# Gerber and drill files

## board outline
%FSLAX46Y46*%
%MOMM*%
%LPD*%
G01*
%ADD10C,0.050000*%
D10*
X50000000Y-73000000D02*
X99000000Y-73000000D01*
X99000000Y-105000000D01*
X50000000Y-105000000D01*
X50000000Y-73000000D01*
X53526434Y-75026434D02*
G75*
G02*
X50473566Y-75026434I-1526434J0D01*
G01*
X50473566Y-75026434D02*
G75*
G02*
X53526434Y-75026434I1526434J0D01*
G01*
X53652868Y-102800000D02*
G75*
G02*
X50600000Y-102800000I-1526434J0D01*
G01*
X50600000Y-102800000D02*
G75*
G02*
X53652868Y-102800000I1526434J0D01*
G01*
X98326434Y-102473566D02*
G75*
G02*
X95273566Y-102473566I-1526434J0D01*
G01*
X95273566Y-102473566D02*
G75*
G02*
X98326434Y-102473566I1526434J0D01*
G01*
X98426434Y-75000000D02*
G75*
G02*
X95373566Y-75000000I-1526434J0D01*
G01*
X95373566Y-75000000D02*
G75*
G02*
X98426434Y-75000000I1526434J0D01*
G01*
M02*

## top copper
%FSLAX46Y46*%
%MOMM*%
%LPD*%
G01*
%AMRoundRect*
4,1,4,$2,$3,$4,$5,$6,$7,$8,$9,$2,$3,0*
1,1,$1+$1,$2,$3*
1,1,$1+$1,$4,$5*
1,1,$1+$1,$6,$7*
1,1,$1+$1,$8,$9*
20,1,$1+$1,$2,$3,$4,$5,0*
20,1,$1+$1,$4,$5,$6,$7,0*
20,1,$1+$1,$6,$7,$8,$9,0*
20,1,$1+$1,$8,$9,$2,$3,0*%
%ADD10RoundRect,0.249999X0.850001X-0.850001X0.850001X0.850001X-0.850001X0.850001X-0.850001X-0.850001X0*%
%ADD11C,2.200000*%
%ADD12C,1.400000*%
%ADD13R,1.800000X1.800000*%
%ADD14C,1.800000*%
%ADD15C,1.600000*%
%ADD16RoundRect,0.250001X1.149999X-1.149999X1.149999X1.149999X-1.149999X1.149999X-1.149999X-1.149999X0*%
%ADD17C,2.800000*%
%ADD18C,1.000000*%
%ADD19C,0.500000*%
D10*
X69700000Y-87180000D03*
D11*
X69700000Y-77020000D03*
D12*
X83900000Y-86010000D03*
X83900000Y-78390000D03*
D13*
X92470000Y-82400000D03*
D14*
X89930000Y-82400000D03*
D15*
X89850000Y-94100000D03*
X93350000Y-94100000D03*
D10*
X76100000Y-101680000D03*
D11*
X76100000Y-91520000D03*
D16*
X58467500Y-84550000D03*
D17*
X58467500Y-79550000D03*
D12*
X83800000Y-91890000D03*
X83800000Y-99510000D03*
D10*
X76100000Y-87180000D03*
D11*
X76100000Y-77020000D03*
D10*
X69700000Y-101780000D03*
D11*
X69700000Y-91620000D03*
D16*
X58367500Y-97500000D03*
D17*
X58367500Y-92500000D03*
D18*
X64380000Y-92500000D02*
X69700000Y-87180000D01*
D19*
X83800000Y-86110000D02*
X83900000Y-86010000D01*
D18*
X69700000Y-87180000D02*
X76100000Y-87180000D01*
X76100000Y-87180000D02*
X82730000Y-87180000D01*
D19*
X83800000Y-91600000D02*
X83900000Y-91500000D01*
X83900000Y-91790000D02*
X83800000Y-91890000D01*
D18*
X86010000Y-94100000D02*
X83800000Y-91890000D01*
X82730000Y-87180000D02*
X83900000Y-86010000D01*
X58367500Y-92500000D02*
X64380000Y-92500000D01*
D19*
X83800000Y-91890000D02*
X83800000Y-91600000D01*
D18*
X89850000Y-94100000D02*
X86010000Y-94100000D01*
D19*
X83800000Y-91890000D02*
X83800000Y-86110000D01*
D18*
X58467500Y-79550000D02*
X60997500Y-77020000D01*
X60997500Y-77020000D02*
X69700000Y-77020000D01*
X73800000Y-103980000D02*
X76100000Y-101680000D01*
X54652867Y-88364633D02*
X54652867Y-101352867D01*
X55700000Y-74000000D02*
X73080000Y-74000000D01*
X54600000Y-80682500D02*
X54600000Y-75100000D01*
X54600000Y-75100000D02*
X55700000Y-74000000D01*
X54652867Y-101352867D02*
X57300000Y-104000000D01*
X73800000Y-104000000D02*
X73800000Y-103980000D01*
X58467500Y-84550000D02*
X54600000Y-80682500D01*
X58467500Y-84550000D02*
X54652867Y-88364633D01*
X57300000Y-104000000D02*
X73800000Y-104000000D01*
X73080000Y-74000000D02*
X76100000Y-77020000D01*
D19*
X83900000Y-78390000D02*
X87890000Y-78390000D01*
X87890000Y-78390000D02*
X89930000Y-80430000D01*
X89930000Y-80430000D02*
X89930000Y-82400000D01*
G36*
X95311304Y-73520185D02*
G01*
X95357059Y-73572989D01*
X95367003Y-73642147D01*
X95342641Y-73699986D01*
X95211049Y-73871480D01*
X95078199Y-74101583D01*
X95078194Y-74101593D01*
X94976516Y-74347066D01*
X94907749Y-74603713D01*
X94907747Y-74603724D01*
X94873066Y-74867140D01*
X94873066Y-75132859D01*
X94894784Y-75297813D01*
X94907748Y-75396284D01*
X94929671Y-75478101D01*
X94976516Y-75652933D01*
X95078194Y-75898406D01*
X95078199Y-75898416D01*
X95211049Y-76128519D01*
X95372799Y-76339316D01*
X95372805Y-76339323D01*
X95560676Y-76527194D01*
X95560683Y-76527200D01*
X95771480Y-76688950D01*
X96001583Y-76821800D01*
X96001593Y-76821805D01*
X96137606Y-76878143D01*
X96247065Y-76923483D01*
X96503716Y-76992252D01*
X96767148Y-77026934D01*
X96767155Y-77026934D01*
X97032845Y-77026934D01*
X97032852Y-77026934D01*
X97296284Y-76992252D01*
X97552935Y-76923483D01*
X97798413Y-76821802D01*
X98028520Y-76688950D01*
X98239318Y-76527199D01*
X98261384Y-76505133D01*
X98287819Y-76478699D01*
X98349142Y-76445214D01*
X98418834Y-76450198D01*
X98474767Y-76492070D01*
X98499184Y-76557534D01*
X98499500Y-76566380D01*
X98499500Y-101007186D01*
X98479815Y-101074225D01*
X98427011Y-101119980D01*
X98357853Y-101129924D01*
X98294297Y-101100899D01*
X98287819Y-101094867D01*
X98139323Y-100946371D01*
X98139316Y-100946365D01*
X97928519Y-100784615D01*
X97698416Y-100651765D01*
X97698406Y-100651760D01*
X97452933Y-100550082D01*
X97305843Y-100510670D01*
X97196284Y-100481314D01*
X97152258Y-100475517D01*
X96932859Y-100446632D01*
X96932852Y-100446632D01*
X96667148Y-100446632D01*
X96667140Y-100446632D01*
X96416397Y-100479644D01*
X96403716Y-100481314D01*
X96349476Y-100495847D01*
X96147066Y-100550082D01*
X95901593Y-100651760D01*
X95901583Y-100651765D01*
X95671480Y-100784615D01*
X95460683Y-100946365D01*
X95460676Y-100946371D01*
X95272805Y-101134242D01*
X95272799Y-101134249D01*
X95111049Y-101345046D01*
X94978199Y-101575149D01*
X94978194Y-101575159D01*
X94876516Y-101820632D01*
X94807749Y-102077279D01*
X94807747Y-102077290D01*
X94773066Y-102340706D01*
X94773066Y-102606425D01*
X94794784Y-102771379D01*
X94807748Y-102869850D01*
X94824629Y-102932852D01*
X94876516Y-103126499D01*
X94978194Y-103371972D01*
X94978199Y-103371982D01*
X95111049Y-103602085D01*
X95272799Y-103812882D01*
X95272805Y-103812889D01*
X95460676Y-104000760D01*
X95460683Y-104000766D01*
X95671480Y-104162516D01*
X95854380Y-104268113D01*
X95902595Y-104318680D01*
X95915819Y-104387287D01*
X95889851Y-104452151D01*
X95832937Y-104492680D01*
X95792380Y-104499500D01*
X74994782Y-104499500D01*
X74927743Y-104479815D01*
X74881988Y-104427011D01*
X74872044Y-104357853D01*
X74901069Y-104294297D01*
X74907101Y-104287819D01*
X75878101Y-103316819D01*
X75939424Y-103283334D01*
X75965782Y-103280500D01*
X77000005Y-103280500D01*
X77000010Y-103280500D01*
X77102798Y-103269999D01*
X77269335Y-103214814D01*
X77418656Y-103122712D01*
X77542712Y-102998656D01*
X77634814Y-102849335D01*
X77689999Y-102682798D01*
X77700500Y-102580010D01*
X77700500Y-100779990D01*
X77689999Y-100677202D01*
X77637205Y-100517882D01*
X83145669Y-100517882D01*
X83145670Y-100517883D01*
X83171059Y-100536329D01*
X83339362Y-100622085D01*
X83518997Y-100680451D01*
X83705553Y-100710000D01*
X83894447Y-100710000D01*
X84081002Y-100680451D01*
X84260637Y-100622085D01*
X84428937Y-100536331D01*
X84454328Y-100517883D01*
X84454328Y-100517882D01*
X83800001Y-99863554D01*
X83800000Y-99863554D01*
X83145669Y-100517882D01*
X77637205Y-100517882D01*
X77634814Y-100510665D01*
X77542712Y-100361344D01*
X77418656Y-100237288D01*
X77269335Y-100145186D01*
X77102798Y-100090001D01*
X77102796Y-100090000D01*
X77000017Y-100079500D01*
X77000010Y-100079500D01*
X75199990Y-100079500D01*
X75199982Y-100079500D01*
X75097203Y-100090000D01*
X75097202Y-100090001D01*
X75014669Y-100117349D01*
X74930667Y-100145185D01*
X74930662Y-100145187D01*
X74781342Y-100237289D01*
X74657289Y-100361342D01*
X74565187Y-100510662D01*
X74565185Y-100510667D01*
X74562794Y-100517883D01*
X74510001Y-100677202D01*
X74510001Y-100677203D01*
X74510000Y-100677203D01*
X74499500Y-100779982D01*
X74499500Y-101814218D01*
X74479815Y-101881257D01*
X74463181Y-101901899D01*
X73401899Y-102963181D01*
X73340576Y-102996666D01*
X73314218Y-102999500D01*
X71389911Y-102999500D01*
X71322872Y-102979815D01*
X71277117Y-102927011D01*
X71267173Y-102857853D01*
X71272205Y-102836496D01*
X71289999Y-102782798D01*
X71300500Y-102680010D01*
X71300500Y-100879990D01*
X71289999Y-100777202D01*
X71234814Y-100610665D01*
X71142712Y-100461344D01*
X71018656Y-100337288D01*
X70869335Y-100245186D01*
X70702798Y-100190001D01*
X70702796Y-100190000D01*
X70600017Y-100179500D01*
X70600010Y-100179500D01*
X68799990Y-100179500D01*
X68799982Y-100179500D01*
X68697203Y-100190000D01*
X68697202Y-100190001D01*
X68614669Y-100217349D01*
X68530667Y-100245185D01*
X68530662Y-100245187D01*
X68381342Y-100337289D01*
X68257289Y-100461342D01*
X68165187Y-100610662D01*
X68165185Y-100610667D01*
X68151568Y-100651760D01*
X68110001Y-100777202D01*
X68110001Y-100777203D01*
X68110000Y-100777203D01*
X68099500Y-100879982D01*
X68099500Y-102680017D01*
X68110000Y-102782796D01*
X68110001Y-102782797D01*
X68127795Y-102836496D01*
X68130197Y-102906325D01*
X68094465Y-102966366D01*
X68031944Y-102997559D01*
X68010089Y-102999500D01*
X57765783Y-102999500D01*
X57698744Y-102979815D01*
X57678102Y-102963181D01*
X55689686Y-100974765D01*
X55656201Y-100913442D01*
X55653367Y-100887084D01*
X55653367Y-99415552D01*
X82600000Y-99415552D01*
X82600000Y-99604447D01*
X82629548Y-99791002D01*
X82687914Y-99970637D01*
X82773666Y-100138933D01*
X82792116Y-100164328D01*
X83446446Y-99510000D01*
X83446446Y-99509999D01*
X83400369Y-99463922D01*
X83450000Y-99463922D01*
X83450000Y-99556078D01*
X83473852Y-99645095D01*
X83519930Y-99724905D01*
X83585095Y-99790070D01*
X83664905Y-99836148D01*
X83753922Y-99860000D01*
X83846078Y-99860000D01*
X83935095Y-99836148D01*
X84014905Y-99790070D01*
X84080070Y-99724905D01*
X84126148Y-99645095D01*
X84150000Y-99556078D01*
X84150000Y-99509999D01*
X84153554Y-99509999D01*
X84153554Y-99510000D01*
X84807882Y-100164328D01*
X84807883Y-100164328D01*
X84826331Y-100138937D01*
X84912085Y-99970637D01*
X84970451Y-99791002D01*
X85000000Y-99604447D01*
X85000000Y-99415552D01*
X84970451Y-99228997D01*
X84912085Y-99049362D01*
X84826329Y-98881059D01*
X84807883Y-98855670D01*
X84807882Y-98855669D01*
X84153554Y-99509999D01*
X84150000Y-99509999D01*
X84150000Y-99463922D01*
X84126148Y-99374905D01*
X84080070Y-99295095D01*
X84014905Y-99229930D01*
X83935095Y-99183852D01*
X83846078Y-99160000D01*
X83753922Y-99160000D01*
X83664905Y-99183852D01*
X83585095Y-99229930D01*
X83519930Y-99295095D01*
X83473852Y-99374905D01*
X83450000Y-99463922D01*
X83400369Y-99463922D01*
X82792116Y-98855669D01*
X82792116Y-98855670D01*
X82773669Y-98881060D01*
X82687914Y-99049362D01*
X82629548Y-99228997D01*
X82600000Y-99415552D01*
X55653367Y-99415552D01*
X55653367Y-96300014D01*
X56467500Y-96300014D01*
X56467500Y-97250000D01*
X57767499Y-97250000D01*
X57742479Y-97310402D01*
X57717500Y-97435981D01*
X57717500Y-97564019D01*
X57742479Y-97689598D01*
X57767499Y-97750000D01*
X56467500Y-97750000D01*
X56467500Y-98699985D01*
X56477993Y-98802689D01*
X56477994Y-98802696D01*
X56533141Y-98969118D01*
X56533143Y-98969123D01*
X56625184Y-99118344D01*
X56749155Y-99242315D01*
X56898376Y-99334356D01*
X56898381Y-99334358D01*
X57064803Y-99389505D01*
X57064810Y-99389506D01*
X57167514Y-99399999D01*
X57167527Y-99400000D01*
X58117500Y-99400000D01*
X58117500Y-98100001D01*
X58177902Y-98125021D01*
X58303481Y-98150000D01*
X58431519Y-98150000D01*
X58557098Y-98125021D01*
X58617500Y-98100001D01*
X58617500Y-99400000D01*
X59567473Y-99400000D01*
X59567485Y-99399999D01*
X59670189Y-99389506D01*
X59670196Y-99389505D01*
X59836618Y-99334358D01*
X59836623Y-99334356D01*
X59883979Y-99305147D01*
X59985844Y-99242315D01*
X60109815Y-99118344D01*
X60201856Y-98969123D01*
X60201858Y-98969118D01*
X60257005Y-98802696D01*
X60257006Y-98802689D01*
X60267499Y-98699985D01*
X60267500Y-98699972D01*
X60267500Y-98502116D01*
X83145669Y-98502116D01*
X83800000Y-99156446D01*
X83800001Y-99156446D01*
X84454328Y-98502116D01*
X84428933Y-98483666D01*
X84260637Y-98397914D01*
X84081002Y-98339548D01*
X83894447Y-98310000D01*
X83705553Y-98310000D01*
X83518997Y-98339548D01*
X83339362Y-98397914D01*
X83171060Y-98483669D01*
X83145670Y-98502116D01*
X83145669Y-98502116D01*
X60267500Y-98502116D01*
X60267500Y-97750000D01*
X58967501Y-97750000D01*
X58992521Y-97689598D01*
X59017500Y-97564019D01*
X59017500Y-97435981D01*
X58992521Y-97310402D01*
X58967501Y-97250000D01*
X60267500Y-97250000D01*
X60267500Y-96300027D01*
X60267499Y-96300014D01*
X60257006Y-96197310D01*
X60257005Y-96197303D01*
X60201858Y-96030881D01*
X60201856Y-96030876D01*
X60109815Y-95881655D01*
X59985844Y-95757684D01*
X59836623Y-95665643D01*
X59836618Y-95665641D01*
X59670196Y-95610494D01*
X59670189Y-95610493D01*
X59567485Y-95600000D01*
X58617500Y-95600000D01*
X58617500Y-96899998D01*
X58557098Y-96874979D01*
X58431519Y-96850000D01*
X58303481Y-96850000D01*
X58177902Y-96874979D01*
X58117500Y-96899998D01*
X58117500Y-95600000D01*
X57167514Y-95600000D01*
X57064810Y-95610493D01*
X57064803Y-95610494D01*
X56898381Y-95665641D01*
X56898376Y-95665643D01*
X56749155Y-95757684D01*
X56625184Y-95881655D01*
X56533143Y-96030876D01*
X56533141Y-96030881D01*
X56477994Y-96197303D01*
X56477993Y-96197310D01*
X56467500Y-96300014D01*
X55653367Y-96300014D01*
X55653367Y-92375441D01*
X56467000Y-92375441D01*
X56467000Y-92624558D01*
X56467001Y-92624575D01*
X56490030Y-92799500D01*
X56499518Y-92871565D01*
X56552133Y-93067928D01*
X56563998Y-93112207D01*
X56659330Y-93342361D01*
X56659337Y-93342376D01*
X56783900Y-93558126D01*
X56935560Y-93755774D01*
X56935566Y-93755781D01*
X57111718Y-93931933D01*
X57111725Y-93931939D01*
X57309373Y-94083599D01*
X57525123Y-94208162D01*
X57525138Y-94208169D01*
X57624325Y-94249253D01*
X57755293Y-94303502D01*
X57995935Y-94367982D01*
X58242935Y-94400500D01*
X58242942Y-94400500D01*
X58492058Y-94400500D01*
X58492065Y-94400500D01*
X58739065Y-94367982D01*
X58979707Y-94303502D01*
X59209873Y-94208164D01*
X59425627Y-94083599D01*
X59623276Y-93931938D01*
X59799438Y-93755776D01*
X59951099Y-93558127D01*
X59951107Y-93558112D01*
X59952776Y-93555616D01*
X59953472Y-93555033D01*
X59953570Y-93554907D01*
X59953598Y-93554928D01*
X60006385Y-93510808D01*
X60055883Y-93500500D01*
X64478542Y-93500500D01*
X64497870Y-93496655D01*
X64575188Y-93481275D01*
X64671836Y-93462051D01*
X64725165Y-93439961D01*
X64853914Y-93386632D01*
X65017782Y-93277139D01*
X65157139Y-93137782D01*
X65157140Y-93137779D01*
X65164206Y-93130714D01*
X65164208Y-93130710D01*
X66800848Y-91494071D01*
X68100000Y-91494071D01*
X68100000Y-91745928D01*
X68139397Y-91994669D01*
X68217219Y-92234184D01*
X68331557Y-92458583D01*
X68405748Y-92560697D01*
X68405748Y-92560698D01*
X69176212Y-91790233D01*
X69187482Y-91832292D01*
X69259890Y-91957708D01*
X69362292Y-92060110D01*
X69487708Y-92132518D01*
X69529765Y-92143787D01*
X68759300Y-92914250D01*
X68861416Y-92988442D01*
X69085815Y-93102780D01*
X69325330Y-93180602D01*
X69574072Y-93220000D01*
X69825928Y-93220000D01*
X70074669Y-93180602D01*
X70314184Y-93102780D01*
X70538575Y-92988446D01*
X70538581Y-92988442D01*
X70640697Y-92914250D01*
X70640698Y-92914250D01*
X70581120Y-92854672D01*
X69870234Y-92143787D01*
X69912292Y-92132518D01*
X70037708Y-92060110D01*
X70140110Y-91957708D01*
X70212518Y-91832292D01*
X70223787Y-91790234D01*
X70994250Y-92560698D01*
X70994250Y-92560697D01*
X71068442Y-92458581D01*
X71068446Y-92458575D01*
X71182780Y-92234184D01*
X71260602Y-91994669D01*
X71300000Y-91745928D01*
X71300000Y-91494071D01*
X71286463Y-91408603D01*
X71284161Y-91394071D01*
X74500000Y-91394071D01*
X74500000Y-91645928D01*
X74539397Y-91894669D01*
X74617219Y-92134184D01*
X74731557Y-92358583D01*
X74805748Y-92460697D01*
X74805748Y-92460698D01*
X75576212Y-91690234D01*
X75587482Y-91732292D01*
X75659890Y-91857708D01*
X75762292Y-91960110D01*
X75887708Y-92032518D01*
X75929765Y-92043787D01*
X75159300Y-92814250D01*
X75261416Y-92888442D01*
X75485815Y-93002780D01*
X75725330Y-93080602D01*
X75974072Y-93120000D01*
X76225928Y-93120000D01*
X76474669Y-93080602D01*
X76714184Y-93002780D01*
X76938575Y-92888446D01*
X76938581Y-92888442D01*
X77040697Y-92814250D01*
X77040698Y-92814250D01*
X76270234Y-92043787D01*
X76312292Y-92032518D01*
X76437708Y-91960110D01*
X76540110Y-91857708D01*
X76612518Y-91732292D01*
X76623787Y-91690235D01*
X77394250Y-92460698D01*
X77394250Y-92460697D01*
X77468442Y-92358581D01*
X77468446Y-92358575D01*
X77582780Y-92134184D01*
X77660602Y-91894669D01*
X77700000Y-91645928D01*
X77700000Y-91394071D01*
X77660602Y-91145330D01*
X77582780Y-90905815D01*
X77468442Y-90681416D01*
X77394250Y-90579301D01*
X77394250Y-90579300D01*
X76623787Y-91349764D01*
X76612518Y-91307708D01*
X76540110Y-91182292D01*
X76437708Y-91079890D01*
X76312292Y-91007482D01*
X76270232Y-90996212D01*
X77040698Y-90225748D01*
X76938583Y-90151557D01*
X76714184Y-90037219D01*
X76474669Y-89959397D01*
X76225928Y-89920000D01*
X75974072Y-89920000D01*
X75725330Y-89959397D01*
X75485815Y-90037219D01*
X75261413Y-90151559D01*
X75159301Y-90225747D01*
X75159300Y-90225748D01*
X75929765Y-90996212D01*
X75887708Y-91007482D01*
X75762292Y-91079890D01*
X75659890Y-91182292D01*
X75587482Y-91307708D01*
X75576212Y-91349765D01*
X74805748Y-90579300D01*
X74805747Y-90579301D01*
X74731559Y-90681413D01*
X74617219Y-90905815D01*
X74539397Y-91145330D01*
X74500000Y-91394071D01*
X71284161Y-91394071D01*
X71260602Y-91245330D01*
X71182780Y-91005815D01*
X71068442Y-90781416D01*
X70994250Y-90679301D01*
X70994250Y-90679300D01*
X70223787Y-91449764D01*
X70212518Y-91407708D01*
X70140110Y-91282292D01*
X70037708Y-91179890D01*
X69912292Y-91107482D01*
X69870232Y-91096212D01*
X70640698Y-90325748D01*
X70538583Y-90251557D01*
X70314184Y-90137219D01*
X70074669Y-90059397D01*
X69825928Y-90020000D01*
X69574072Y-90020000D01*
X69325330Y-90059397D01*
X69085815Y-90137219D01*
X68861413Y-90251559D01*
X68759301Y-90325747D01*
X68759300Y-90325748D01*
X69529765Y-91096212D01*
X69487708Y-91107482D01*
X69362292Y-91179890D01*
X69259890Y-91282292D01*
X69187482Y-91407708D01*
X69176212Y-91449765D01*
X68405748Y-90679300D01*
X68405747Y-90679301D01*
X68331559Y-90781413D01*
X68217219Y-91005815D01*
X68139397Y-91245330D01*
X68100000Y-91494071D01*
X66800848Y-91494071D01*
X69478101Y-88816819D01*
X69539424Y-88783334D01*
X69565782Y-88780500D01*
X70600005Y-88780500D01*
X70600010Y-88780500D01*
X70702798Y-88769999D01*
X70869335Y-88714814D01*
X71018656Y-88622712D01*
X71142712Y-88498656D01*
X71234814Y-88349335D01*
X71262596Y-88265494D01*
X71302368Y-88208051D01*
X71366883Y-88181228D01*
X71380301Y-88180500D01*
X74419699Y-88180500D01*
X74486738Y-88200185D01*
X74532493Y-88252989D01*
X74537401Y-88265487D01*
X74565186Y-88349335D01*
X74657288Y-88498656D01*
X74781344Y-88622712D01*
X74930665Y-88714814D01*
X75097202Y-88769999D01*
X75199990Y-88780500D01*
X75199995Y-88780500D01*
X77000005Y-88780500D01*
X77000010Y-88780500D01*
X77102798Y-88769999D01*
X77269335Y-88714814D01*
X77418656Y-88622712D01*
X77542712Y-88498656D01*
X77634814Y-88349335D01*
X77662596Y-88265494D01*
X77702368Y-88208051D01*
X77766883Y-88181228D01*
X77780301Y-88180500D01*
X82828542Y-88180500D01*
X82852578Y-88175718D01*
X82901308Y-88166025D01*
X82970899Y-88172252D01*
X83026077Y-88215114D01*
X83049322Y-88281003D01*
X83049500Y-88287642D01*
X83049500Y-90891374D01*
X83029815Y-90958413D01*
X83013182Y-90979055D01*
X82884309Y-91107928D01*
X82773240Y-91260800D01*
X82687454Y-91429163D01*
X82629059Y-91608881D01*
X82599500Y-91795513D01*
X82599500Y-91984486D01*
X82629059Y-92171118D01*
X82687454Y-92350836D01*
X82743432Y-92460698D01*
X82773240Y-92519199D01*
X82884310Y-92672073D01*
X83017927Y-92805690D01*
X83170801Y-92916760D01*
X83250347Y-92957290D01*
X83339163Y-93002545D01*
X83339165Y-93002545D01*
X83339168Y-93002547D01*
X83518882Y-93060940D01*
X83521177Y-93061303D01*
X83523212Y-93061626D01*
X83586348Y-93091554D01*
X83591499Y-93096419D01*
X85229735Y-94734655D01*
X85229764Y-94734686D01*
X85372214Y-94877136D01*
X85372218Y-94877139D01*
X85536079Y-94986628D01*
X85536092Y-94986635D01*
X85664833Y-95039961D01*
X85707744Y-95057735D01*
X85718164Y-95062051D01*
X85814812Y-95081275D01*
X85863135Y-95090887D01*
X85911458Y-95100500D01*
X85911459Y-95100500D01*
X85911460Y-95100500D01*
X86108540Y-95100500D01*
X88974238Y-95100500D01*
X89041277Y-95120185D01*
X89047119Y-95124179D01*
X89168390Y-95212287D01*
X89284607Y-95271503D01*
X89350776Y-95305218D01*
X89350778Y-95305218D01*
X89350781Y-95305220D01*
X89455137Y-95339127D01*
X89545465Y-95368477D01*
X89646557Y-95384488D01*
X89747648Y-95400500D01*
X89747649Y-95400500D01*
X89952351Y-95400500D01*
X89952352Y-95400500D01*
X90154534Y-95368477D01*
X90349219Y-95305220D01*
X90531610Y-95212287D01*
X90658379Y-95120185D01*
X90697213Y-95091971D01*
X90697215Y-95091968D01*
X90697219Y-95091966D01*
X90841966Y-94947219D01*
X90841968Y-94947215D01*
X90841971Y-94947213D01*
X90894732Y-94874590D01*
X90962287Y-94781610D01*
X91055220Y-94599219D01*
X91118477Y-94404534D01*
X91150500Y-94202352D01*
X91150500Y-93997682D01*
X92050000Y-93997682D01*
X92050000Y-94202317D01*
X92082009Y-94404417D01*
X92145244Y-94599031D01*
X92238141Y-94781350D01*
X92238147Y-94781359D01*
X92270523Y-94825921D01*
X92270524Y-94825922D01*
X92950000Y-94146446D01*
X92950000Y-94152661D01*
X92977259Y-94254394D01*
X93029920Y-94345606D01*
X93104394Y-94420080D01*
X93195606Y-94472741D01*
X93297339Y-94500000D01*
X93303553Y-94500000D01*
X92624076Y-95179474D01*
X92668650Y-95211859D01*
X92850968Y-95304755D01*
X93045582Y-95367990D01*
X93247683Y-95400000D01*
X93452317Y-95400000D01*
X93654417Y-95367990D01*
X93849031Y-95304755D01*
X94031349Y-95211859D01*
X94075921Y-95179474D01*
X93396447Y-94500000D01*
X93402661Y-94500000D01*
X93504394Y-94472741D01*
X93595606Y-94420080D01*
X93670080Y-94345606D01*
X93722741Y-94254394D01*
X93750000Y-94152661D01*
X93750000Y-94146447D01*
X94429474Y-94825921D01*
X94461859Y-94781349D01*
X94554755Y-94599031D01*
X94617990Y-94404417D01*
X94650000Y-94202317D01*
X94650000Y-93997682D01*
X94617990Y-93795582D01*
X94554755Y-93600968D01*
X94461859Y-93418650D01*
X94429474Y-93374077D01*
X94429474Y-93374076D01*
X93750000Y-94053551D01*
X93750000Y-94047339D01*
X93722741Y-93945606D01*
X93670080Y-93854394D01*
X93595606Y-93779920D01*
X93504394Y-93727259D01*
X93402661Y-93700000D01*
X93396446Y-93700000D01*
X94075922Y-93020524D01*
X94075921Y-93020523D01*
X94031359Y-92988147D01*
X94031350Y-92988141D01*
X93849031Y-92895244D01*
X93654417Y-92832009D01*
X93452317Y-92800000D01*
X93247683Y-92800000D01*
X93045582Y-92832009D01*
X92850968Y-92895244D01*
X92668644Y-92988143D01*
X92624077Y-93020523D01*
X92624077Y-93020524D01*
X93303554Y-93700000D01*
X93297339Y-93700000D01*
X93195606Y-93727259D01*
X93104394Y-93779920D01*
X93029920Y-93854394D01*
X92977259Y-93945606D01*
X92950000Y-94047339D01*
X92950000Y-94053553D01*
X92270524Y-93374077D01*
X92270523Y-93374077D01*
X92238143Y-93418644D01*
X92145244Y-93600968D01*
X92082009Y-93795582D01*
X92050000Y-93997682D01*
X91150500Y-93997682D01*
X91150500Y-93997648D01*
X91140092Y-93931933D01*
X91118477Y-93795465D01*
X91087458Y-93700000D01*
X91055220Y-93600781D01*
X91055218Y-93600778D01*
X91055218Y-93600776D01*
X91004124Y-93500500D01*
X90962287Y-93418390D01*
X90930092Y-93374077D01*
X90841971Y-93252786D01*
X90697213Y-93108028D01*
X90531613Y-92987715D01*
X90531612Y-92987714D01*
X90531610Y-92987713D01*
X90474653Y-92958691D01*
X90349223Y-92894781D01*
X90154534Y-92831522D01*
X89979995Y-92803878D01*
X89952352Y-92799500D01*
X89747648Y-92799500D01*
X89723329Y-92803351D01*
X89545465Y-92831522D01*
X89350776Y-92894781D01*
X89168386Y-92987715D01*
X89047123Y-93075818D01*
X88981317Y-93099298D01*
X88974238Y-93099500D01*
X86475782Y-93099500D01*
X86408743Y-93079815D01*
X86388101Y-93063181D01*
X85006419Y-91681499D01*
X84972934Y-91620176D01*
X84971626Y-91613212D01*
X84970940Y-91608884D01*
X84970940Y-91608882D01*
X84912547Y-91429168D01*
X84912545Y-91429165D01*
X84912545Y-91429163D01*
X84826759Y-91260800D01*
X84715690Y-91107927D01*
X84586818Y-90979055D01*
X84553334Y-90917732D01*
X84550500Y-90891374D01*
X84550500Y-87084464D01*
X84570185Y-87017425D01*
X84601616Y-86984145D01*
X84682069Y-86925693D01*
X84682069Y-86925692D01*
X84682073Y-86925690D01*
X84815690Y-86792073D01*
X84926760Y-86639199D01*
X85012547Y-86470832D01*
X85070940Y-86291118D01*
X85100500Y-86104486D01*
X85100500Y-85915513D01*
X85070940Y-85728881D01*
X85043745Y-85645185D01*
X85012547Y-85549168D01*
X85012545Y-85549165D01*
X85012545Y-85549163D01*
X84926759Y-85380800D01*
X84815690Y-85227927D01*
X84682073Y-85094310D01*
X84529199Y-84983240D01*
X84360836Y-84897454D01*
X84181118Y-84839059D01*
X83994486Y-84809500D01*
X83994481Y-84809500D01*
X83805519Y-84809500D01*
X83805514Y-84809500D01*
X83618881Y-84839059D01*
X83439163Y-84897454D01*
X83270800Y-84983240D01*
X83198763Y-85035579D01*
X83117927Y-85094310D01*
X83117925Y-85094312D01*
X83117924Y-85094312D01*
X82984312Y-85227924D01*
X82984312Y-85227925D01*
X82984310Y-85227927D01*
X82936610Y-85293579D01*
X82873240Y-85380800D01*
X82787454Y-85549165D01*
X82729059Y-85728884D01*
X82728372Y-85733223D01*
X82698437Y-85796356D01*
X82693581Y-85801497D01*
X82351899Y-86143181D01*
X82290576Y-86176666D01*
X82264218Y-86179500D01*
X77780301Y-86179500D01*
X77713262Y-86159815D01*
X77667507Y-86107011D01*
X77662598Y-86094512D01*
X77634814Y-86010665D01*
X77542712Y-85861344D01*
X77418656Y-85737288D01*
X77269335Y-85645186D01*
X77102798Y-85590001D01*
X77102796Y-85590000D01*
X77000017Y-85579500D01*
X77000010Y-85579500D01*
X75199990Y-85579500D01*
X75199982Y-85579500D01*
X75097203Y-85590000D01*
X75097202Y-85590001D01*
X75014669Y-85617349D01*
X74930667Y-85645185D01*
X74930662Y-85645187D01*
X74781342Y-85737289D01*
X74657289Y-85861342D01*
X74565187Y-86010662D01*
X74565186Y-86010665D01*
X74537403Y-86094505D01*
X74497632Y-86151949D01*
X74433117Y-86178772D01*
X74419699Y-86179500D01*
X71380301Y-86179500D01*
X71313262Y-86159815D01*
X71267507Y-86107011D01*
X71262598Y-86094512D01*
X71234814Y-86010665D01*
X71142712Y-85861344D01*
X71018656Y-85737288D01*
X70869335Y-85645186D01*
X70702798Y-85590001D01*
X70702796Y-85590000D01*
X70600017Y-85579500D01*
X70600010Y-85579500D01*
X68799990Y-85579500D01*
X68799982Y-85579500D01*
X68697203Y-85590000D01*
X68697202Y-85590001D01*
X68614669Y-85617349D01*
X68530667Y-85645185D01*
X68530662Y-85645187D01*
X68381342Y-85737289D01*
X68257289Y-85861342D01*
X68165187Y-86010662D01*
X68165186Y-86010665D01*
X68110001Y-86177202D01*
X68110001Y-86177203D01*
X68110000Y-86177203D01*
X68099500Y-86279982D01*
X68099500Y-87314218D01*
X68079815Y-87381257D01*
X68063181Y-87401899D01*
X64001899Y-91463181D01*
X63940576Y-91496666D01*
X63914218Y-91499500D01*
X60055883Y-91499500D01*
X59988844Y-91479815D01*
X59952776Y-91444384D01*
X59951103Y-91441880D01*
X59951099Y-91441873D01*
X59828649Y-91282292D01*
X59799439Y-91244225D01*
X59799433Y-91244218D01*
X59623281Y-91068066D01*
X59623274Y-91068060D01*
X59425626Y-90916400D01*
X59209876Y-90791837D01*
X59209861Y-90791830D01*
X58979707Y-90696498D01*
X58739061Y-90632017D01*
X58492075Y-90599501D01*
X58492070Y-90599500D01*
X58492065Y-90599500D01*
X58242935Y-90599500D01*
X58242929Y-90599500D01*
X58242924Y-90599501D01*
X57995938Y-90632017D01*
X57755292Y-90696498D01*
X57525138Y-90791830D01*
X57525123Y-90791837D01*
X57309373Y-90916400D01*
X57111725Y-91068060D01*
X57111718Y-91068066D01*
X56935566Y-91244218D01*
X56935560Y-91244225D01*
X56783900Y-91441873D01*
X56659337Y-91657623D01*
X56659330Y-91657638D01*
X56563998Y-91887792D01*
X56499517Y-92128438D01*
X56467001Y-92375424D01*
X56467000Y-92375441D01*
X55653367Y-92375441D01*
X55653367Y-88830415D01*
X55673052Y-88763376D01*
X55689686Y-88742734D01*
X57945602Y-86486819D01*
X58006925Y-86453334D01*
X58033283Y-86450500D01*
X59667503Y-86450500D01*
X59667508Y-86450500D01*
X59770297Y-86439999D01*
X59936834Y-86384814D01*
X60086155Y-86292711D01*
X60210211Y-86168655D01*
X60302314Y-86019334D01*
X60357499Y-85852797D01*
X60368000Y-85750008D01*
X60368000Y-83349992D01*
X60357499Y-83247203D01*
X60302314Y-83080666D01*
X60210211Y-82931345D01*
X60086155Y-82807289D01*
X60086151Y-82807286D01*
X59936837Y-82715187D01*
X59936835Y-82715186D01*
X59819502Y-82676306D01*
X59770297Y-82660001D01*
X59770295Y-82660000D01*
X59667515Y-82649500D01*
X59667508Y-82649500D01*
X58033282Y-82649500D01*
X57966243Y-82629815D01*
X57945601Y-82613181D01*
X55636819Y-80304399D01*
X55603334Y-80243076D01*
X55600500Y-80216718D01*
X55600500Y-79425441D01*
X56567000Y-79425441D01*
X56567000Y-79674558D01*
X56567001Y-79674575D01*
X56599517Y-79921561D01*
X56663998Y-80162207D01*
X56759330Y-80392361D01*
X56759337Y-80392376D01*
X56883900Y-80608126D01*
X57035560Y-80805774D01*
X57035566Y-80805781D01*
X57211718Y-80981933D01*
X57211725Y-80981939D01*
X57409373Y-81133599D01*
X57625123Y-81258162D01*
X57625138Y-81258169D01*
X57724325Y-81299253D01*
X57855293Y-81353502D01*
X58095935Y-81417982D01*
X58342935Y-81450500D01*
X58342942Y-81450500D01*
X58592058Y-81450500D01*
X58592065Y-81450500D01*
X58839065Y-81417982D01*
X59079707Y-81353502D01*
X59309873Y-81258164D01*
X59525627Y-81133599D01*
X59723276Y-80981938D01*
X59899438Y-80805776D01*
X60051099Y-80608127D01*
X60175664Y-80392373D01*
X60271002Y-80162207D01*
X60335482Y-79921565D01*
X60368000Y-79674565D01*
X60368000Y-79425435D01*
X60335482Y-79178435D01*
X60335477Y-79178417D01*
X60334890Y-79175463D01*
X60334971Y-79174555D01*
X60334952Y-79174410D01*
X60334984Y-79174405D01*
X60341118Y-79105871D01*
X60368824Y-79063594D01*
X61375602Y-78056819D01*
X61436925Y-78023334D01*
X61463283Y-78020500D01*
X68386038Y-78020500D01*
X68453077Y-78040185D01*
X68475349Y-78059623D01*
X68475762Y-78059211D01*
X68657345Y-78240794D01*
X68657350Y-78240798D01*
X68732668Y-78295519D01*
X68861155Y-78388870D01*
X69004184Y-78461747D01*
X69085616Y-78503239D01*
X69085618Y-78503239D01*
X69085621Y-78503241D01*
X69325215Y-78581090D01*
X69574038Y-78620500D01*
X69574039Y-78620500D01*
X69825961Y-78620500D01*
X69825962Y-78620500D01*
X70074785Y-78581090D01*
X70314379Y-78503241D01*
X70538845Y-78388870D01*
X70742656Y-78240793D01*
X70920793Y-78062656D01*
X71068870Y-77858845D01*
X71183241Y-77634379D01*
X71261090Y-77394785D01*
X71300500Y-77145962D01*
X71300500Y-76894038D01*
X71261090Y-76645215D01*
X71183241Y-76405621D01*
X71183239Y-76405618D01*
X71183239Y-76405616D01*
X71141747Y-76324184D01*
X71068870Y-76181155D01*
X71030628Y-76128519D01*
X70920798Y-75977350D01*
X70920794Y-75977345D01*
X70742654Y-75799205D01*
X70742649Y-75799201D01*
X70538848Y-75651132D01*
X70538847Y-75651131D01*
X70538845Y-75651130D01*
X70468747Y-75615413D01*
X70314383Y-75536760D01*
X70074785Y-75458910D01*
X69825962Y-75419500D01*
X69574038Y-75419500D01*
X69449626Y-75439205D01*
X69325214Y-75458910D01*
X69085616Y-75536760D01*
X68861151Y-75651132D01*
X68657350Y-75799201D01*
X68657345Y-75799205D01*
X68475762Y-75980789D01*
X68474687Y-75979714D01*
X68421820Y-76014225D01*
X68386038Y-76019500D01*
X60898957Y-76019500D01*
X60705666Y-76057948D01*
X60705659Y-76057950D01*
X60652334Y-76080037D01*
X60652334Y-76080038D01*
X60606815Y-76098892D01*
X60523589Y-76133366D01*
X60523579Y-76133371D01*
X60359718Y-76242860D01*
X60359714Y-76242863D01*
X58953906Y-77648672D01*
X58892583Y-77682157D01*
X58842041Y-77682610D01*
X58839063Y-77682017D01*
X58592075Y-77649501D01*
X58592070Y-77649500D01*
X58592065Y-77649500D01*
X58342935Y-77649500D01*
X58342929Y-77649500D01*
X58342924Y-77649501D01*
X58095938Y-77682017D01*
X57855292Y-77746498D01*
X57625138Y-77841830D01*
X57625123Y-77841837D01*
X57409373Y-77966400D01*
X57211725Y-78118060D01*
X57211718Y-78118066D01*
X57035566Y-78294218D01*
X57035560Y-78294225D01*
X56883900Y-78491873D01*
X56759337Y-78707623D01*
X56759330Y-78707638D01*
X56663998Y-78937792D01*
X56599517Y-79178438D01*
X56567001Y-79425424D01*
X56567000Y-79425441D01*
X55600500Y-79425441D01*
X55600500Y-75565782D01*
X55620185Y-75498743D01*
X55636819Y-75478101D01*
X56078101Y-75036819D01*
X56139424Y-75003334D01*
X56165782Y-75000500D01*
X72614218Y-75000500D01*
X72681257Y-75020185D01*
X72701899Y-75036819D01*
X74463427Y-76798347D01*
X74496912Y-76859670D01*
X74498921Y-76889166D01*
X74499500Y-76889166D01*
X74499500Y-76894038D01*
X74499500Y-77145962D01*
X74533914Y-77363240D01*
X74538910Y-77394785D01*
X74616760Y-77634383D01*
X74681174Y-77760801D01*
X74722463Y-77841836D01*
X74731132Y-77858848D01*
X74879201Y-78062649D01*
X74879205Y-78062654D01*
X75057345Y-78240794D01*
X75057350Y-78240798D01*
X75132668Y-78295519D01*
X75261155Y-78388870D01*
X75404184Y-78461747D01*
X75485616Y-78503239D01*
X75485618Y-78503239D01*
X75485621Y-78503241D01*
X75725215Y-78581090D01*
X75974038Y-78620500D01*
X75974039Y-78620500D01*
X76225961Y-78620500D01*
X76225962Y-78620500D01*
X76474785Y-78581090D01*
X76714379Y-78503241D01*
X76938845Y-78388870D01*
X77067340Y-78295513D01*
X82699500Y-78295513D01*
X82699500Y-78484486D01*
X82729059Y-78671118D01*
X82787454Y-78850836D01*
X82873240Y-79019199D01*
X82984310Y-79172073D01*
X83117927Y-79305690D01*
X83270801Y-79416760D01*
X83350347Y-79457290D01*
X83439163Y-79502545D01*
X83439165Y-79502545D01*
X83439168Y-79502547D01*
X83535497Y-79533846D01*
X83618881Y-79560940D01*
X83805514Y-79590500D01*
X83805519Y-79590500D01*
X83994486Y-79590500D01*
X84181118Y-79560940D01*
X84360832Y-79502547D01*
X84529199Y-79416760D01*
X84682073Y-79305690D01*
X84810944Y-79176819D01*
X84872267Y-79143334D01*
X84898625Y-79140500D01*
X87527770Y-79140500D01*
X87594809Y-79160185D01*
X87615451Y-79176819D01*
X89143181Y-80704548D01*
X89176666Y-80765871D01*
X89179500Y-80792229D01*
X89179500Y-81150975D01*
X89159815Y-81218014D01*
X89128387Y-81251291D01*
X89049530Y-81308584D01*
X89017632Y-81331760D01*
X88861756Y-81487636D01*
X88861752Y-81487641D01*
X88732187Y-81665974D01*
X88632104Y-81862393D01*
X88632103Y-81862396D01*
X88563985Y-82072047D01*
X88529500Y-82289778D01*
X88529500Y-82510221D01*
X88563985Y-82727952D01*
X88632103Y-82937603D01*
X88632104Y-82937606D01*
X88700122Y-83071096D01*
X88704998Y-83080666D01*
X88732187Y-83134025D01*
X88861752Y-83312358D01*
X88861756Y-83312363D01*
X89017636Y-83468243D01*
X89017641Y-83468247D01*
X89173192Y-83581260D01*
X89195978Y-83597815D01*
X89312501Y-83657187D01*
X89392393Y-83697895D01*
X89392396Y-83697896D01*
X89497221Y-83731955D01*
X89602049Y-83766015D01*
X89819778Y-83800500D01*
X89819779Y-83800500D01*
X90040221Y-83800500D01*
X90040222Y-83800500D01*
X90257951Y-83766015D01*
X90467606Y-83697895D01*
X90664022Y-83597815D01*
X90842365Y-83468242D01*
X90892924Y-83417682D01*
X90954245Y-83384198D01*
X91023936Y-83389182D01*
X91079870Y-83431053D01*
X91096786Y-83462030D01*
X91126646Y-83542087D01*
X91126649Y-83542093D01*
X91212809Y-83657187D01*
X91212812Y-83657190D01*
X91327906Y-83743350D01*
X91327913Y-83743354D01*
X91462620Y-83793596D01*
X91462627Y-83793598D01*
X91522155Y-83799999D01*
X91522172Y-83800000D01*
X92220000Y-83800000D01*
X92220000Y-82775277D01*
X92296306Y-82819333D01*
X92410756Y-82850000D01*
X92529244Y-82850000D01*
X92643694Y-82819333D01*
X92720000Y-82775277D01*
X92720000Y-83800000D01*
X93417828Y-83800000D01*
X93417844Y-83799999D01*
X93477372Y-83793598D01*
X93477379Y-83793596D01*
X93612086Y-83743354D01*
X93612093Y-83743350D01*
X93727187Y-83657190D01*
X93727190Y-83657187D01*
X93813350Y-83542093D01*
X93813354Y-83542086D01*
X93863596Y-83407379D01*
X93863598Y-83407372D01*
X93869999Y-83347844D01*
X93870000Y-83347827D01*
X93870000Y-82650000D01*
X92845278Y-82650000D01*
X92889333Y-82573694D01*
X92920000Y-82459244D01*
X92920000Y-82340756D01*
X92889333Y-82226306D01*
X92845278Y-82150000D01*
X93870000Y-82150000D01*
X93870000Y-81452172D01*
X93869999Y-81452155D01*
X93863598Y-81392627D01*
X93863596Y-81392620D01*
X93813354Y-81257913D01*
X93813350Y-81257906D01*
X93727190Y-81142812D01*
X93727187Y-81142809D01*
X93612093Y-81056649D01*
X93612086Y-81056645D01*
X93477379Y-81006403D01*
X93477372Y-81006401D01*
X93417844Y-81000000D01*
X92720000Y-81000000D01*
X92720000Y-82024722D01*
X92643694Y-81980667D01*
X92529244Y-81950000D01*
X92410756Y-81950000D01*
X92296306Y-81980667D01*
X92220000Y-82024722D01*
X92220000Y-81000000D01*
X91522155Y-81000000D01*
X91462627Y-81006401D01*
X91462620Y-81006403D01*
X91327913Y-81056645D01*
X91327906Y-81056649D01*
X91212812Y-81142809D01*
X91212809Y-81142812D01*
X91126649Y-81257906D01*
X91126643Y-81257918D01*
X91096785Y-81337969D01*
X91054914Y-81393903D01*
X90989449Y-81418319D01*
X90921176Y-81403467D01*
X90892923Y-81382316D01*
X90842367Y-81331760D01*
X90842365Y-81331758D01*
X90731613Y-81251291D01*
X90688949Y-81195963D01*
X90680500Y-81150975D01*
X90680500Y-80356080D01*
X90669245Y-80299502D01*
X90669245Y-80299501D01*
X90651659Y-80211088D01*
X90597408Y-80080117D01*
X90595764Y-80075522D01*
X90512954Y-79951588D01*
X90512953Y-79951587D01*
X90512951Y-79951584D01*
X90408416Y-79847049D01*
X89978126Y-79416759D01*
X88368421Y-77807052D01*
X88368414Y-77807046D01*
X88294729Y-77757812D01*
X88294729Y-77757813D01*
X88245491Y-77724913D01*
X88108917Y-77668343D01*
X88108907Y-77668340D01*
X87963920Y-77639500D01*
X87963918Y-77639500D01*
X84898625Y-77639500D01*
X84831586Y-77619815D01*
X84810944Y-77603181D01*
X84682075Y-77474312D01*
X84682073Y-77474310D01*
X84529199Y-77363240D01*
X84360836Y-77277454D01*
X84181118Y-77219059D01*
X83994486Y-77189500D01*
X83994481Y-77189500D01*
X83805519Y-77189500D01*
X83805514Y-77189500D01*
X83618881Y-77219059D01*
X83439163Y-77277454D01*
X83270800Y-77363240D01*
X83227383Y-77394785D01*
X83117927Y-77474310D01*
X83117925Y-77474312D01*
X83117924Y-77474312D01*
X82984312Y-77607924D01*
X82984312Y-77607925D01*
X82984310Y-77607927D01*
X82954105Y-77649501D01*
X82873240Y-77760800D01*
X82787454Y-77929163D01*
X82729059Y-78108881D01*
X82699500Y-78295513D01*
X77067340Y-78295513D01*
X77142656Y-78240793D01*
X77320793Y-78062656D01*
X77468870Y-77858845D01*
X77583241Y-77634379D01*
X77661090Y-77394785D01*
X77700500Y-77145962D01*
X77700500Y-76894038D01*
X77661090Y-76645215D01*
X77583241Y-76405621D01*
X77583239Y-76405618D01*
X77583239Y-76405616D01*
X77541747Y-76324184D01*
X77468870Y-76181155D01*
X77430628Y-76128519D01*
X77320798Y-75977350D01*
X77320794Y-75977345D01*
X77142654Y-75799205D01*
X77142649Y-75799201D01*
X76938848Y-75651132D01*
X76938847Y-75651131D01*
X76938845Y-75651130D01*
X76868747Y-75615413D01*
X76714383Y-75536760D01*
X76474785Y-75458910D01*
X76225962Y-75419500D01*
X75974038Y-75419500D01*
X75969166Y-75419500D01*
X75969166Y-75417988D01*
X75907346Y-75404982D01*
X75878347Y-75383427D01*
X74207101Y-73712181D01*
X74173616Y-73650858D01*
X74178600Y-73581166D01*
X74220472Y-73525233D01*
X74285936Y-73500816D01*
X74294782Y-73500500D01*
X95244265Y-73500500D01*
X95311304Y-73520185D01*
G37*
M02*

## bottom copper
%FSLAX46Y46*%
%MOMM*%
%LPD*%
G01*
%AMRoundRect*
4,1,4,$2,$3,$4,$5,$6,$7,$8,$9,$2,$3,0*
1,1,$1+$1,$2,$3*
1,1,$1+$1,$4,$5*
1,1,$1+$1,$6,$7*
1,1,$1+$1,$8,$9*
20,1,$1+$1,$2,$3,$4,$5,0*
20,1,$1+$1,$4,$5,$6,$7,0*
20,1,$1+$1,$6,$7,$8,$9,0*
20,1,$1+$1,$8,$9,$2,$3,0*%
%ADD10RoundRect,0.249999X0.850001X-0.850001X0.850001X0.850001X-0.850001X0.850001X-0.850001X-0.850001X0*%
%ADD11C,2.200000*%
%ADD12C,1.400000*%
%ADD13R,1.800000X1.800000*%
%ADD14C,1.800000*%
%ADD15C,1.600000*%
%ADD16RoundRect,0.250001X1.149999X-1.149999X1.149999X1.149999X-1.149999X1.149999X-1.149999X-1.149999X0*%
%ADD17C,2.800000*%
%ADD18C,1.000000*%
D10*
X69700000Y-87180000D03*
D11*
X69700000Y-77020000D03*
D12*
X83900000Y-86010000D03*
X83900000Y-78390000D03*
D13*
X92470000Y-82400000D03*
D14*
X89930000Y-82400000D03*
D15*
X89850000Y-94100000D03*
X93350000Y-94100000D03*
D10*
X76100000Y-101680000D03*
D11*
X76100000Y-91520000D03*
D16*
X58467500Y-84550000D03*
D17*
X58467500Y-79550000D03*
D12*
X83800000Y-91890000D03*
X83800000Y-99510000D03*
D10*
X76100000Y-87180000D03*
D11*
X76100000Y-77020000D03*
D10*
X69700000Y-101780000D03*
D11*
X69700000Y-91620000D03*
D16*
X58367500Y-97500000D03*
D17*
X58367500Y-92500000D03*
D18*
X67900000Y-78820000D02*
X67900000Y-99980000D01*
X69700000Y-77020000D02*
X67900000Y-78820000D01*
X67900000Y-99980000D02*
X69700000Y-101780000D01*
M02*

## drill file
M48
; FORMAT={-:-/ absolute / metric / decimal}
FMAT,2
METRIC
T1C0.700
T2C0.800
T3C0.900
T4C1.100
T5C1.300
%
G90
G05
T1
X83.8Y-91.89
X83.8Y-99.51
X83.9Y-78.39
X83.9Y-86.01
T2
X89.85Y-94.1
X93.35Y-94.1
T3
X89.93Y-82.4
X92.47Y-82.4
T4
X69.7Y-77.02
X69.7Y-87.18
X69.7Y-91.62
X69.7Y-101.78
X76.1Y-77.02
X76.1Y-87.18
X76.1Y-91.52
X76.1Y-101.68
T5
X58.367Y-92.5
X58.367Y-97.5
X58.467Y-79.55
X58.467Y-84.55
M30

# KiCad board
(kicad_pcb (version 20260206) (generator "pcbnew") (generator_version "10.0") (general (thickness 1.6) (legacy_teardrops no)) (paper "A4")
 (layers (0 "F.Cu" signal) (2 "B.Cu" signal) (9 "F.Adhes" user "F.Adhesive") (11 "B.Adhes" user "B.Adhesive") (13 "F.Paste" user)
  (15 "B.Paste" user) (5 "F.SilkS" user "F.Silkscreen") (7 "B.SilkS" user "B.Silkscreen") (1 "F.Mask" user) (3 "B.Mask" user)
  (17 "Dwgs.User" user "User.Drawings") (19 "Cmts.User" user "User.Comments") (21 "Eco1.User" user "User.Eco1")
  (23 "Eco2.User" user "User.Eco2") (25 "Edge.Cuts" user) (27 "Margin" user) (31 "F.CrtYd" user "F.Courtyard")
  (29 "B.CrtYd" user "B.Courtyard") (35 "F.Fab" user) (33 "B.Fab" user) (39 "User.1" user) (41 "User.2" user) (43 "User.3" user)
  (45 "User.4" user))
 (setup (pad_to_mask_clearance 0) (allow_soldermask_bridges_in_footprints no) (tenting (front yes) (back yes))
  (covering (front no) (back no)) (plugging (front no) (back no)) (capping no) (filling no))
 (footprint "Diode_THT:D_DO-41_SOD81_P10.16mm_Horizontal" (layer "F.Cu") (at 69.7 87.18 90)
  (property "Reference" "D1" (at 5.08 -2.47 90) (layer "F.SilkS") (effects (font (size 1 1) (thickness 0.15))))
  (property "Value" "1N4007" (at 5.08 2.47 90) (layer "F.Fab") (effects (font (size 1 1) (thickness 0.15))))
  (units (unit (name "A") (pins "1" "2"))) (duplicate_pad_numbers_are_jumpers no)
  (pad "1" thru_hole roundrect (at 0 0 90) (size 2.2 2.2) (drill 1.1) (layers "*.Cu" "*.Mask") (remove_unused_layers no)
   (roundrect_rratio 0.113636) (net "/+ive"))
  (pad "2" thru_hole circle (at 10.16 0 90) (size 2.2 2.2) (drill 1.1) (layers "*.Cu" "*.Mask") (remove_unused_layers no) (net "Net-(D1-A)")))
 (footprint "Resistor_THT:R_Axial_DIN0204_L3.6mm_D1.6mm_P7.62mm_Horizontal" (layer "F.Cu") (at 83.9 86.01 90)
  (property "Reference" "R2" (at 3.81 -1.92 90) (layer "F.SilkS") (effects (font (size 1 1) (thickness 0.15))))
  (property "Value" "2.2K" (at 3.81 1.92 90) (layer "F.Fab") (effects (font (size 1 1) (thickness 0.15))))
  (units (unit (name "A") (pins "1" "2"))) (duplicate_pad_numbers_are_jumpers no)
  (pad "1" thru_hole circle (at 0 0 90) (size 1.4 1.4) (drill 0.7) (layers "*.Cu" "*.Mask") (remove_unused_layers no) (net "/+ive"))
  (pad "2" thru_hole circle (at 7.62 0 90) (size 1.4 1.4) (drill 0.7) (layers "*.Cu" "*.Mask") (remove_unused_layers no) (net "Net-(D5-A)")))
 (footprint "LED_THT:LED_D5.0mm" (layer "F.Cu") (at 92.47 82.4 180)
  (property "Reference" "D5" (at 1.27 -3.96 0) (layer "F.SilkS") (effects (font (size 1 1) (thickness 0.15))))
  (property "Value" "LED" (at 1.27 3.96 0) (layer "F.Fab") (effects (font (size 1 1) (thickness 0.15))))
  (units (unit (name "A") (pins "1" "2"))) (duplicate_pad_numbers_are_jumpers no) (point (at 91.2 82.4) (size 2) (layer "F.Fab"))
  (pad "1" thru_hole rect (at 0 0 180) (size 1.8 1.8) (drill 0.9) (layers "*.Cu" "*.Mask") (remove_unused_layers no) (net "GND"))
  (pad "2" thru_hole circle (at 2.54 0 180) (size 1.8 1.8) (drill 0.9) (layers "*.Cu" "*.Mask") (remove_unused_layers no) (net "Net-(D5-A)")))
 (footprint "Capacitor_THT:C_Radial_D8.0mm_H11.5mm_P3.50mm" (layer "F.Cu") (at 89.85 94.1)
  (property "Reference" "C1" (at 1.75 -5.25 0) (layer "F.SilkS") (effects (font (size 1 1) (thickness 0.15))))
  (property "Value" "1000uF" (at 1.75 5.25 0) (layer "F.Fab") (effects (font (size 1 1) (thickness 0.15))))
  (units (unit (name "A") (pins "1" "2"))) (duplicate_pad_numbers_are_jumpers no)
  (pad "1" thru_hole circle (at 0 0) (size 1.6 1.6) (drill 0.8) (layers "*.Cu" "*.Mask") (remove_unused_layers no) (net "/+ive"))
  (pad "2" thru_hole circle (at 3.5 0) (size 1.6 1.6) (drill 0.8) (layers "*.Cu" "*.Mask") (remove_unused_layers no) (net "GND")))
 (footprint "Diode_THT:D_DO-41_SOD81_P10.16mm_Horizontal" (layer "F.Cu") (at 76.1 101.68 90)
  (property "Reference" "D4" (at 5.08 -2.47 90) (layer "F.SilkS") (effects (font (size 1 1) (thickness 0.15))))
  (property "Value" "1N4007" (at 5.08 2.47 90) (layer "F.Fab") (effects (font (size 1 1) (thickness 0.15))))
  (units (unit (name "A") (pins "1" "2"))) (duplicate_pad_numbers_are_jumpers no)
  (pad "1" thru_hole roundrect (at 0 0 90) (size 2.2 2.2) (drill 1.1) (layers "*.Cu" "*.Mask") (remove_unused_layers no)
   (roundrect_rratio 0.113636) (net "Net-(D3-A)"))
  (pad "2" thru_hole circle (at 10.16 0 90) (size 2.2 2.2) (drill 1.1) (layers "*.Cu" "*.Mask") (remove_unused_layers no) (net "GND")))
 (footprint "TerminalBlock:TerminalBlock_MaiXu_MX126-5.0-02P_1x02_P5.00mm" (layer "F.Cu") (at 58.4675 84.55 90)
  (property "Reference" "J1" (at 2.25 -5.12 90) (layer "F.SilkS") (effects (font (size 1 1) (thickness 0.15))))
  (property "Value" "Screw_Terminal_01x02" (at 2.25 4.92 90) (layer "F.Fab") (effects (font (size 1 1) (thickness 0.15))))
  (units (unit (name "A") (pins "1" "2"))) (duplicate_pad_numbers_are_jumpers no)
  (pad "1" thru_hole roundrect (at 0 0 90) (size 2.8 2.8) (drill 1.3) (layers "*.Cu" "*.Mask") (remove_unused_layers no)
   (roundrect_rratio 0.089286) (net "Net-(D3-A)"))
  (pad "2" thru_hole circle (at 5 0 90) (size 2.8 2.8) (drill 1.3) (layers "*.Cu" "*.Mask") (remove_unused_layers no) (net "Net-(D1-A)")))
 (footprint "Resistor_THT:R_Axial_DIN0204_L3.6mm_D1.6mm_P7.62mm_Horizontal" (layer "F.Cu") (at 83.8 91.89 -90)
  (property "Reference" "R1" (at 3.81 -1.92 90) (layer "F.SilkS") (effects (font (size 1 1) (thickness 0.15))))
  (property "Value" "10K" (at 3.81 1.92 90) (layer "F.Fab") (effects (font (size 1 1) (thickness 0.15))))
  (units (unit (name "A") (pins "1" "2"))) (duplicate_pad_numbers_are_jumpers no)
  (pad "1" thru_hole circle (at 0 0 270) (size 1.4 1.4) (drill 0.7) (layers "*.Cu" "*.Mask") (remove_unused_layers no) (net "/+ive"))
  (pad "2" thru_hole circle (at 7.62 0 270) (size 1.4 1.4) (drill 0.7) (layers "*.Cu" "*.Mask") (remove_unused_layers no) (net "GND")))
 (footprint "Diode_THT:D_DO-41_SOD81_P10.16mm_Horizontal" (layer "F.Cu") (at 76.1 87.18 90)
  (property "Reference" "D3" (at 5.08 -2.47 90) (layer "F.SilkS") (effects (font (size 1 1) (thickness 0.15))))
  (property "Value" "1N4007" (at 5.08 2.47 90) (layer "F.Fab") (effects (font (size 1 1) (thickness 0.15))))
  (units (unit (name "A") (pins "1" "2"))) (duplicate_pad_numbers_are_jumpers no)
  (pad "1" thru_hole roundrect (at 0 0 90) (size 2.2 2.2) (drill 1.1) (layers "*.Cu" "*.Mask") (remove_unused_layers no)
   (roundrect_rratio 0.113636) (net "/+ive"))
  (pad "2" thru_hole circle (at 10.16 0 90) (size 2.2 2.2) (drill 1.1) (layers "*.Cu" "*.Mask") (remove_unused_layers no) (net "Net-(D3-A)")))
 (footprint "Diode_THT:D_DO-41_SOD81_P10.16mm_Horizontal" (layer "F.Cu") (at 69.7 101.78 90)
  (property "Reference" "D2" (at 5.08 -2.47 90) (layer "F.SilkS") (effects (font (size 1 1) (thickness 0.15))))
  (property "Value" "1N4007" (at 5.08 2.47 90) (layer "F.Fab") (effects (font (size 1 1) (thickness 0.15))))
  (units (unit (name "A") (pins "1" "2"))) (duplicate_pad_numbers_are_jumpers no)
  (pad "1" thru_hole roundrect (at 0 0 90) (size 2.2 2.2) (drill 1.1) (layers "*.Cu" "*.Mask") (remove_unused_layers no)
   (roundrect_rratio 0.113636) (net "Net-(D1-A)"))
  (pad "2" thru_hole circle (at 10.16 0 90) (size 2.2 2.2) (drill 1.1) (layers "*.Cu" "*.Mask") (remove_unused_layers no) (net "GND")))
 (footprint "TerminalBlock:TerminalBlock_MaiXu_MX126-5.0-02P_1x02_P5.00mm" (layer "F.Cu") (at 58.3675 97.5 90)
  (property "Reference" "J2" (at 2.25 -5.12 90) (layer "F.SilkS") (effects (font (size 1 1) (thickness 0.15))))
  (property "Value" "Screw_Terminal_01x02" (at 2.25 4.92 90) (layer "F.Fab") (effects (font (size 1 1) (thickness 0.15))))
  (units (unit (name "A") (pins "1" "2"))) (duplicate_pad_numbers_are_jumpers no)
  (pad "1" thru_hole roundrect (at 0 0 90) (size 2.8 2.8) (drill 1.3) (layers "*.Cu" "*.Mask") (remove_unused_layers no)
   (roundrect_rratio 0.089286) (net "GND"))
  (pad "2" thru_hole circle (at 5 0 90) (size 2.8 2.8) (drill 1.3) (layers "*.Cu" "*.Mask") (remove_unused_layers no) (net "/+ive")))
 (gr_rect (start 50 73) (end 99 105) (stroke (width 0.05) (type default)) (fill no) (layer "Edge.Cuts"))
 (gr_circle (center 52 75.026434) (end 53.3 74.226434) (stroke (width 0.05) (type default)) (fill no) (layer "Edge.Cuts"))
 (gr_circle (center 52.126434 102.8) (end 53.426434 102) (stroke (width 0.05) (type default)) (fill no) (layer "Edge.Cuts"))
 (gr_circle (center 96.8 102.473566) (end 98.1 101.673566) (stroke (width 0.05) (type default)) (fill no) (layer "Edge.Cuts"))
 (gr_circle (center 96.9 75) (end 98.2 74.2) (stroke (width 0.05) (type default)) (fill no) (layer "Edge.Cuts"))
 (segment (start 64.38 92.5) (end 69.7 87.18) (width 1) (layer "F.Cu") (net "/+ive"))
 (segment (start 83.8 86.11) (end 83.9 86.01) (width 0.5) (layer "F.Cu") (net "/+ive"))
 (segment (start 69.7 87.18) (end 76.1 87.18) (width 1) (layer "F.Cu") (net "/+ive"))
 (segment (start 76.1 87.18) (end 82.73 87.18) (width 1) (layer "F.Cu") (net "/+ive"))
 (segment (start 83.8 91.6) (end 83.9 91.5) (width 0.5) (layer "F.Cu") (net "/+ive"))
 (segment (start 83.9 91.79) (end 83.8 91.89) (width 0.5) (layer "F.Cu") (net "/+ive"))
 (segment (start 86.01 94.1) (end 83.8 91.89) (width 1) (layer "F.Cu") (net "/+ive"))
 (segment (start 82.73 87.18) (end 83.9 86.01) (width 1) (layer "F.Cu") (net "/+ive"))
 (segment (start 58.3675 92.5) (end 64.38 92.5) (width 1) (layer "F.Cu") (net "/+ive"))
 (segment (start 83.8 91.89) (end 83.8 91.6) (width 0.5) (layer "F.Cu") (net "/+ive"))
 (segment (start 89.85 94.1) (end 86.01 94.1) (width 1) (layer "F.Cu") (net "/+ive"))
 (segment (start 83.8 91.89) (end 83.8 86.11) (width 0.5) (layer "F.Cu") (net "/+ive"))
 (segment (start 58.4675 79.55) (end 60.9975 77.02) (width 1) (layer "F.Cu") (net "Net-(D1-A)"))
 (segment (start 60.9975 77.02) (end 69.7 77.02) (width 1) (layer "F.Cu") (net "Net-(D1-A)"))
 (segment (start 67.9 78.82) (end 67.9 99.98) (width 1) (layer "B.Cu") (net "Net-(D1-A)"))
 (segment (start 69.7 77.02) (end 67.9 78.82) (width 1) (layer "B.Cu") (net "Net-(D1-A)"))
 (segment (start 67.9 99.98) (end 69.7 101.78) (width 1) (layer "B.Cu") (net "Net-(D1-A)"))
 (segment (start 73.8 103.98) (end 76.1 101.68) (width 1) (layer "F.Cu") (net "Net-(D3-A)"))
 (segment (start 54.652867 88.364633) (end 54.652867 101.352867) (width 1) (layer "F.Cu") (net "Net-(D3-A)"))
 (segment (start 55.7 74) (end 73.08 74) (width 1) (layer "F.Cu") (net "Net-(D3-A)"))
 (segment (start 54.6 80.6825) (end 54.6 75.1) (width 1) (layer "F.Cu") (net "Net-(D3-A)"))
 (segment (start 54.6 75.1) (end 55.7 74) (width 1) (layer "F.Cu") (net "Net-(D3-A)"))
 (segment (start 54.652867 101.352867) (end 57.3 104) (width 1) (layer "F.Cu") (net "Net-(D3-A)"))
 (segment (start 73.8 104) (end 73.8 103.98) (width 1) (layer "F.Cu") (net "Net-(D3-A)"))
 (segment (start 58.4675 84.55) (end 54.6 80.6825) (width 1) (layer "F.Cu") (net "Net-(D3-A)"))
 (segment (start 58.4675 84.55) (end 54.652867 88.364633) (width 1) (layer "F.Cu") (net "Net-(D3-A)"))
 (segment (start 57.3 104) (end 73.8 104) (width 1) (layer "F.Cu") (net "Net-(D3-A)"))
 (segment (start 73.08 74) (end 76.1 77.02) (width 1) (layer "F.Cu") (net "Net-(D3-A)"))
 (segment (start 83.9 78.39) (end 87.89 78.39) (width 0.5) (layer "F.Cu") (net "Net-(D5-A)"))
 (segment (start 87.89 78.39) (end 89.93 80.43) (width 0.5) (layer "F.Cu") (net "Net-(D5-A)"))
 (segment (start 89.93 80.43) (end 89.93 82.4) (width 0.5) (layer "F.Cu") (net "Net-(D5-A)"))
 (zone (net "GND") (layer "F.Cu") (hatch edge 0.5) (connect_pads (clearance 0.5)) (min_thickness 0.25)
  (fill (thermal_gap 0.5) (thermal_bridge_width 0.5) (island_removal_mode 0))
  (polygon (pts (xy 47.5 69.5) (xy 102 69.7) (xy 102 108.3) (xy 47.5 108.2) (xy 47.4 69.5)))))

